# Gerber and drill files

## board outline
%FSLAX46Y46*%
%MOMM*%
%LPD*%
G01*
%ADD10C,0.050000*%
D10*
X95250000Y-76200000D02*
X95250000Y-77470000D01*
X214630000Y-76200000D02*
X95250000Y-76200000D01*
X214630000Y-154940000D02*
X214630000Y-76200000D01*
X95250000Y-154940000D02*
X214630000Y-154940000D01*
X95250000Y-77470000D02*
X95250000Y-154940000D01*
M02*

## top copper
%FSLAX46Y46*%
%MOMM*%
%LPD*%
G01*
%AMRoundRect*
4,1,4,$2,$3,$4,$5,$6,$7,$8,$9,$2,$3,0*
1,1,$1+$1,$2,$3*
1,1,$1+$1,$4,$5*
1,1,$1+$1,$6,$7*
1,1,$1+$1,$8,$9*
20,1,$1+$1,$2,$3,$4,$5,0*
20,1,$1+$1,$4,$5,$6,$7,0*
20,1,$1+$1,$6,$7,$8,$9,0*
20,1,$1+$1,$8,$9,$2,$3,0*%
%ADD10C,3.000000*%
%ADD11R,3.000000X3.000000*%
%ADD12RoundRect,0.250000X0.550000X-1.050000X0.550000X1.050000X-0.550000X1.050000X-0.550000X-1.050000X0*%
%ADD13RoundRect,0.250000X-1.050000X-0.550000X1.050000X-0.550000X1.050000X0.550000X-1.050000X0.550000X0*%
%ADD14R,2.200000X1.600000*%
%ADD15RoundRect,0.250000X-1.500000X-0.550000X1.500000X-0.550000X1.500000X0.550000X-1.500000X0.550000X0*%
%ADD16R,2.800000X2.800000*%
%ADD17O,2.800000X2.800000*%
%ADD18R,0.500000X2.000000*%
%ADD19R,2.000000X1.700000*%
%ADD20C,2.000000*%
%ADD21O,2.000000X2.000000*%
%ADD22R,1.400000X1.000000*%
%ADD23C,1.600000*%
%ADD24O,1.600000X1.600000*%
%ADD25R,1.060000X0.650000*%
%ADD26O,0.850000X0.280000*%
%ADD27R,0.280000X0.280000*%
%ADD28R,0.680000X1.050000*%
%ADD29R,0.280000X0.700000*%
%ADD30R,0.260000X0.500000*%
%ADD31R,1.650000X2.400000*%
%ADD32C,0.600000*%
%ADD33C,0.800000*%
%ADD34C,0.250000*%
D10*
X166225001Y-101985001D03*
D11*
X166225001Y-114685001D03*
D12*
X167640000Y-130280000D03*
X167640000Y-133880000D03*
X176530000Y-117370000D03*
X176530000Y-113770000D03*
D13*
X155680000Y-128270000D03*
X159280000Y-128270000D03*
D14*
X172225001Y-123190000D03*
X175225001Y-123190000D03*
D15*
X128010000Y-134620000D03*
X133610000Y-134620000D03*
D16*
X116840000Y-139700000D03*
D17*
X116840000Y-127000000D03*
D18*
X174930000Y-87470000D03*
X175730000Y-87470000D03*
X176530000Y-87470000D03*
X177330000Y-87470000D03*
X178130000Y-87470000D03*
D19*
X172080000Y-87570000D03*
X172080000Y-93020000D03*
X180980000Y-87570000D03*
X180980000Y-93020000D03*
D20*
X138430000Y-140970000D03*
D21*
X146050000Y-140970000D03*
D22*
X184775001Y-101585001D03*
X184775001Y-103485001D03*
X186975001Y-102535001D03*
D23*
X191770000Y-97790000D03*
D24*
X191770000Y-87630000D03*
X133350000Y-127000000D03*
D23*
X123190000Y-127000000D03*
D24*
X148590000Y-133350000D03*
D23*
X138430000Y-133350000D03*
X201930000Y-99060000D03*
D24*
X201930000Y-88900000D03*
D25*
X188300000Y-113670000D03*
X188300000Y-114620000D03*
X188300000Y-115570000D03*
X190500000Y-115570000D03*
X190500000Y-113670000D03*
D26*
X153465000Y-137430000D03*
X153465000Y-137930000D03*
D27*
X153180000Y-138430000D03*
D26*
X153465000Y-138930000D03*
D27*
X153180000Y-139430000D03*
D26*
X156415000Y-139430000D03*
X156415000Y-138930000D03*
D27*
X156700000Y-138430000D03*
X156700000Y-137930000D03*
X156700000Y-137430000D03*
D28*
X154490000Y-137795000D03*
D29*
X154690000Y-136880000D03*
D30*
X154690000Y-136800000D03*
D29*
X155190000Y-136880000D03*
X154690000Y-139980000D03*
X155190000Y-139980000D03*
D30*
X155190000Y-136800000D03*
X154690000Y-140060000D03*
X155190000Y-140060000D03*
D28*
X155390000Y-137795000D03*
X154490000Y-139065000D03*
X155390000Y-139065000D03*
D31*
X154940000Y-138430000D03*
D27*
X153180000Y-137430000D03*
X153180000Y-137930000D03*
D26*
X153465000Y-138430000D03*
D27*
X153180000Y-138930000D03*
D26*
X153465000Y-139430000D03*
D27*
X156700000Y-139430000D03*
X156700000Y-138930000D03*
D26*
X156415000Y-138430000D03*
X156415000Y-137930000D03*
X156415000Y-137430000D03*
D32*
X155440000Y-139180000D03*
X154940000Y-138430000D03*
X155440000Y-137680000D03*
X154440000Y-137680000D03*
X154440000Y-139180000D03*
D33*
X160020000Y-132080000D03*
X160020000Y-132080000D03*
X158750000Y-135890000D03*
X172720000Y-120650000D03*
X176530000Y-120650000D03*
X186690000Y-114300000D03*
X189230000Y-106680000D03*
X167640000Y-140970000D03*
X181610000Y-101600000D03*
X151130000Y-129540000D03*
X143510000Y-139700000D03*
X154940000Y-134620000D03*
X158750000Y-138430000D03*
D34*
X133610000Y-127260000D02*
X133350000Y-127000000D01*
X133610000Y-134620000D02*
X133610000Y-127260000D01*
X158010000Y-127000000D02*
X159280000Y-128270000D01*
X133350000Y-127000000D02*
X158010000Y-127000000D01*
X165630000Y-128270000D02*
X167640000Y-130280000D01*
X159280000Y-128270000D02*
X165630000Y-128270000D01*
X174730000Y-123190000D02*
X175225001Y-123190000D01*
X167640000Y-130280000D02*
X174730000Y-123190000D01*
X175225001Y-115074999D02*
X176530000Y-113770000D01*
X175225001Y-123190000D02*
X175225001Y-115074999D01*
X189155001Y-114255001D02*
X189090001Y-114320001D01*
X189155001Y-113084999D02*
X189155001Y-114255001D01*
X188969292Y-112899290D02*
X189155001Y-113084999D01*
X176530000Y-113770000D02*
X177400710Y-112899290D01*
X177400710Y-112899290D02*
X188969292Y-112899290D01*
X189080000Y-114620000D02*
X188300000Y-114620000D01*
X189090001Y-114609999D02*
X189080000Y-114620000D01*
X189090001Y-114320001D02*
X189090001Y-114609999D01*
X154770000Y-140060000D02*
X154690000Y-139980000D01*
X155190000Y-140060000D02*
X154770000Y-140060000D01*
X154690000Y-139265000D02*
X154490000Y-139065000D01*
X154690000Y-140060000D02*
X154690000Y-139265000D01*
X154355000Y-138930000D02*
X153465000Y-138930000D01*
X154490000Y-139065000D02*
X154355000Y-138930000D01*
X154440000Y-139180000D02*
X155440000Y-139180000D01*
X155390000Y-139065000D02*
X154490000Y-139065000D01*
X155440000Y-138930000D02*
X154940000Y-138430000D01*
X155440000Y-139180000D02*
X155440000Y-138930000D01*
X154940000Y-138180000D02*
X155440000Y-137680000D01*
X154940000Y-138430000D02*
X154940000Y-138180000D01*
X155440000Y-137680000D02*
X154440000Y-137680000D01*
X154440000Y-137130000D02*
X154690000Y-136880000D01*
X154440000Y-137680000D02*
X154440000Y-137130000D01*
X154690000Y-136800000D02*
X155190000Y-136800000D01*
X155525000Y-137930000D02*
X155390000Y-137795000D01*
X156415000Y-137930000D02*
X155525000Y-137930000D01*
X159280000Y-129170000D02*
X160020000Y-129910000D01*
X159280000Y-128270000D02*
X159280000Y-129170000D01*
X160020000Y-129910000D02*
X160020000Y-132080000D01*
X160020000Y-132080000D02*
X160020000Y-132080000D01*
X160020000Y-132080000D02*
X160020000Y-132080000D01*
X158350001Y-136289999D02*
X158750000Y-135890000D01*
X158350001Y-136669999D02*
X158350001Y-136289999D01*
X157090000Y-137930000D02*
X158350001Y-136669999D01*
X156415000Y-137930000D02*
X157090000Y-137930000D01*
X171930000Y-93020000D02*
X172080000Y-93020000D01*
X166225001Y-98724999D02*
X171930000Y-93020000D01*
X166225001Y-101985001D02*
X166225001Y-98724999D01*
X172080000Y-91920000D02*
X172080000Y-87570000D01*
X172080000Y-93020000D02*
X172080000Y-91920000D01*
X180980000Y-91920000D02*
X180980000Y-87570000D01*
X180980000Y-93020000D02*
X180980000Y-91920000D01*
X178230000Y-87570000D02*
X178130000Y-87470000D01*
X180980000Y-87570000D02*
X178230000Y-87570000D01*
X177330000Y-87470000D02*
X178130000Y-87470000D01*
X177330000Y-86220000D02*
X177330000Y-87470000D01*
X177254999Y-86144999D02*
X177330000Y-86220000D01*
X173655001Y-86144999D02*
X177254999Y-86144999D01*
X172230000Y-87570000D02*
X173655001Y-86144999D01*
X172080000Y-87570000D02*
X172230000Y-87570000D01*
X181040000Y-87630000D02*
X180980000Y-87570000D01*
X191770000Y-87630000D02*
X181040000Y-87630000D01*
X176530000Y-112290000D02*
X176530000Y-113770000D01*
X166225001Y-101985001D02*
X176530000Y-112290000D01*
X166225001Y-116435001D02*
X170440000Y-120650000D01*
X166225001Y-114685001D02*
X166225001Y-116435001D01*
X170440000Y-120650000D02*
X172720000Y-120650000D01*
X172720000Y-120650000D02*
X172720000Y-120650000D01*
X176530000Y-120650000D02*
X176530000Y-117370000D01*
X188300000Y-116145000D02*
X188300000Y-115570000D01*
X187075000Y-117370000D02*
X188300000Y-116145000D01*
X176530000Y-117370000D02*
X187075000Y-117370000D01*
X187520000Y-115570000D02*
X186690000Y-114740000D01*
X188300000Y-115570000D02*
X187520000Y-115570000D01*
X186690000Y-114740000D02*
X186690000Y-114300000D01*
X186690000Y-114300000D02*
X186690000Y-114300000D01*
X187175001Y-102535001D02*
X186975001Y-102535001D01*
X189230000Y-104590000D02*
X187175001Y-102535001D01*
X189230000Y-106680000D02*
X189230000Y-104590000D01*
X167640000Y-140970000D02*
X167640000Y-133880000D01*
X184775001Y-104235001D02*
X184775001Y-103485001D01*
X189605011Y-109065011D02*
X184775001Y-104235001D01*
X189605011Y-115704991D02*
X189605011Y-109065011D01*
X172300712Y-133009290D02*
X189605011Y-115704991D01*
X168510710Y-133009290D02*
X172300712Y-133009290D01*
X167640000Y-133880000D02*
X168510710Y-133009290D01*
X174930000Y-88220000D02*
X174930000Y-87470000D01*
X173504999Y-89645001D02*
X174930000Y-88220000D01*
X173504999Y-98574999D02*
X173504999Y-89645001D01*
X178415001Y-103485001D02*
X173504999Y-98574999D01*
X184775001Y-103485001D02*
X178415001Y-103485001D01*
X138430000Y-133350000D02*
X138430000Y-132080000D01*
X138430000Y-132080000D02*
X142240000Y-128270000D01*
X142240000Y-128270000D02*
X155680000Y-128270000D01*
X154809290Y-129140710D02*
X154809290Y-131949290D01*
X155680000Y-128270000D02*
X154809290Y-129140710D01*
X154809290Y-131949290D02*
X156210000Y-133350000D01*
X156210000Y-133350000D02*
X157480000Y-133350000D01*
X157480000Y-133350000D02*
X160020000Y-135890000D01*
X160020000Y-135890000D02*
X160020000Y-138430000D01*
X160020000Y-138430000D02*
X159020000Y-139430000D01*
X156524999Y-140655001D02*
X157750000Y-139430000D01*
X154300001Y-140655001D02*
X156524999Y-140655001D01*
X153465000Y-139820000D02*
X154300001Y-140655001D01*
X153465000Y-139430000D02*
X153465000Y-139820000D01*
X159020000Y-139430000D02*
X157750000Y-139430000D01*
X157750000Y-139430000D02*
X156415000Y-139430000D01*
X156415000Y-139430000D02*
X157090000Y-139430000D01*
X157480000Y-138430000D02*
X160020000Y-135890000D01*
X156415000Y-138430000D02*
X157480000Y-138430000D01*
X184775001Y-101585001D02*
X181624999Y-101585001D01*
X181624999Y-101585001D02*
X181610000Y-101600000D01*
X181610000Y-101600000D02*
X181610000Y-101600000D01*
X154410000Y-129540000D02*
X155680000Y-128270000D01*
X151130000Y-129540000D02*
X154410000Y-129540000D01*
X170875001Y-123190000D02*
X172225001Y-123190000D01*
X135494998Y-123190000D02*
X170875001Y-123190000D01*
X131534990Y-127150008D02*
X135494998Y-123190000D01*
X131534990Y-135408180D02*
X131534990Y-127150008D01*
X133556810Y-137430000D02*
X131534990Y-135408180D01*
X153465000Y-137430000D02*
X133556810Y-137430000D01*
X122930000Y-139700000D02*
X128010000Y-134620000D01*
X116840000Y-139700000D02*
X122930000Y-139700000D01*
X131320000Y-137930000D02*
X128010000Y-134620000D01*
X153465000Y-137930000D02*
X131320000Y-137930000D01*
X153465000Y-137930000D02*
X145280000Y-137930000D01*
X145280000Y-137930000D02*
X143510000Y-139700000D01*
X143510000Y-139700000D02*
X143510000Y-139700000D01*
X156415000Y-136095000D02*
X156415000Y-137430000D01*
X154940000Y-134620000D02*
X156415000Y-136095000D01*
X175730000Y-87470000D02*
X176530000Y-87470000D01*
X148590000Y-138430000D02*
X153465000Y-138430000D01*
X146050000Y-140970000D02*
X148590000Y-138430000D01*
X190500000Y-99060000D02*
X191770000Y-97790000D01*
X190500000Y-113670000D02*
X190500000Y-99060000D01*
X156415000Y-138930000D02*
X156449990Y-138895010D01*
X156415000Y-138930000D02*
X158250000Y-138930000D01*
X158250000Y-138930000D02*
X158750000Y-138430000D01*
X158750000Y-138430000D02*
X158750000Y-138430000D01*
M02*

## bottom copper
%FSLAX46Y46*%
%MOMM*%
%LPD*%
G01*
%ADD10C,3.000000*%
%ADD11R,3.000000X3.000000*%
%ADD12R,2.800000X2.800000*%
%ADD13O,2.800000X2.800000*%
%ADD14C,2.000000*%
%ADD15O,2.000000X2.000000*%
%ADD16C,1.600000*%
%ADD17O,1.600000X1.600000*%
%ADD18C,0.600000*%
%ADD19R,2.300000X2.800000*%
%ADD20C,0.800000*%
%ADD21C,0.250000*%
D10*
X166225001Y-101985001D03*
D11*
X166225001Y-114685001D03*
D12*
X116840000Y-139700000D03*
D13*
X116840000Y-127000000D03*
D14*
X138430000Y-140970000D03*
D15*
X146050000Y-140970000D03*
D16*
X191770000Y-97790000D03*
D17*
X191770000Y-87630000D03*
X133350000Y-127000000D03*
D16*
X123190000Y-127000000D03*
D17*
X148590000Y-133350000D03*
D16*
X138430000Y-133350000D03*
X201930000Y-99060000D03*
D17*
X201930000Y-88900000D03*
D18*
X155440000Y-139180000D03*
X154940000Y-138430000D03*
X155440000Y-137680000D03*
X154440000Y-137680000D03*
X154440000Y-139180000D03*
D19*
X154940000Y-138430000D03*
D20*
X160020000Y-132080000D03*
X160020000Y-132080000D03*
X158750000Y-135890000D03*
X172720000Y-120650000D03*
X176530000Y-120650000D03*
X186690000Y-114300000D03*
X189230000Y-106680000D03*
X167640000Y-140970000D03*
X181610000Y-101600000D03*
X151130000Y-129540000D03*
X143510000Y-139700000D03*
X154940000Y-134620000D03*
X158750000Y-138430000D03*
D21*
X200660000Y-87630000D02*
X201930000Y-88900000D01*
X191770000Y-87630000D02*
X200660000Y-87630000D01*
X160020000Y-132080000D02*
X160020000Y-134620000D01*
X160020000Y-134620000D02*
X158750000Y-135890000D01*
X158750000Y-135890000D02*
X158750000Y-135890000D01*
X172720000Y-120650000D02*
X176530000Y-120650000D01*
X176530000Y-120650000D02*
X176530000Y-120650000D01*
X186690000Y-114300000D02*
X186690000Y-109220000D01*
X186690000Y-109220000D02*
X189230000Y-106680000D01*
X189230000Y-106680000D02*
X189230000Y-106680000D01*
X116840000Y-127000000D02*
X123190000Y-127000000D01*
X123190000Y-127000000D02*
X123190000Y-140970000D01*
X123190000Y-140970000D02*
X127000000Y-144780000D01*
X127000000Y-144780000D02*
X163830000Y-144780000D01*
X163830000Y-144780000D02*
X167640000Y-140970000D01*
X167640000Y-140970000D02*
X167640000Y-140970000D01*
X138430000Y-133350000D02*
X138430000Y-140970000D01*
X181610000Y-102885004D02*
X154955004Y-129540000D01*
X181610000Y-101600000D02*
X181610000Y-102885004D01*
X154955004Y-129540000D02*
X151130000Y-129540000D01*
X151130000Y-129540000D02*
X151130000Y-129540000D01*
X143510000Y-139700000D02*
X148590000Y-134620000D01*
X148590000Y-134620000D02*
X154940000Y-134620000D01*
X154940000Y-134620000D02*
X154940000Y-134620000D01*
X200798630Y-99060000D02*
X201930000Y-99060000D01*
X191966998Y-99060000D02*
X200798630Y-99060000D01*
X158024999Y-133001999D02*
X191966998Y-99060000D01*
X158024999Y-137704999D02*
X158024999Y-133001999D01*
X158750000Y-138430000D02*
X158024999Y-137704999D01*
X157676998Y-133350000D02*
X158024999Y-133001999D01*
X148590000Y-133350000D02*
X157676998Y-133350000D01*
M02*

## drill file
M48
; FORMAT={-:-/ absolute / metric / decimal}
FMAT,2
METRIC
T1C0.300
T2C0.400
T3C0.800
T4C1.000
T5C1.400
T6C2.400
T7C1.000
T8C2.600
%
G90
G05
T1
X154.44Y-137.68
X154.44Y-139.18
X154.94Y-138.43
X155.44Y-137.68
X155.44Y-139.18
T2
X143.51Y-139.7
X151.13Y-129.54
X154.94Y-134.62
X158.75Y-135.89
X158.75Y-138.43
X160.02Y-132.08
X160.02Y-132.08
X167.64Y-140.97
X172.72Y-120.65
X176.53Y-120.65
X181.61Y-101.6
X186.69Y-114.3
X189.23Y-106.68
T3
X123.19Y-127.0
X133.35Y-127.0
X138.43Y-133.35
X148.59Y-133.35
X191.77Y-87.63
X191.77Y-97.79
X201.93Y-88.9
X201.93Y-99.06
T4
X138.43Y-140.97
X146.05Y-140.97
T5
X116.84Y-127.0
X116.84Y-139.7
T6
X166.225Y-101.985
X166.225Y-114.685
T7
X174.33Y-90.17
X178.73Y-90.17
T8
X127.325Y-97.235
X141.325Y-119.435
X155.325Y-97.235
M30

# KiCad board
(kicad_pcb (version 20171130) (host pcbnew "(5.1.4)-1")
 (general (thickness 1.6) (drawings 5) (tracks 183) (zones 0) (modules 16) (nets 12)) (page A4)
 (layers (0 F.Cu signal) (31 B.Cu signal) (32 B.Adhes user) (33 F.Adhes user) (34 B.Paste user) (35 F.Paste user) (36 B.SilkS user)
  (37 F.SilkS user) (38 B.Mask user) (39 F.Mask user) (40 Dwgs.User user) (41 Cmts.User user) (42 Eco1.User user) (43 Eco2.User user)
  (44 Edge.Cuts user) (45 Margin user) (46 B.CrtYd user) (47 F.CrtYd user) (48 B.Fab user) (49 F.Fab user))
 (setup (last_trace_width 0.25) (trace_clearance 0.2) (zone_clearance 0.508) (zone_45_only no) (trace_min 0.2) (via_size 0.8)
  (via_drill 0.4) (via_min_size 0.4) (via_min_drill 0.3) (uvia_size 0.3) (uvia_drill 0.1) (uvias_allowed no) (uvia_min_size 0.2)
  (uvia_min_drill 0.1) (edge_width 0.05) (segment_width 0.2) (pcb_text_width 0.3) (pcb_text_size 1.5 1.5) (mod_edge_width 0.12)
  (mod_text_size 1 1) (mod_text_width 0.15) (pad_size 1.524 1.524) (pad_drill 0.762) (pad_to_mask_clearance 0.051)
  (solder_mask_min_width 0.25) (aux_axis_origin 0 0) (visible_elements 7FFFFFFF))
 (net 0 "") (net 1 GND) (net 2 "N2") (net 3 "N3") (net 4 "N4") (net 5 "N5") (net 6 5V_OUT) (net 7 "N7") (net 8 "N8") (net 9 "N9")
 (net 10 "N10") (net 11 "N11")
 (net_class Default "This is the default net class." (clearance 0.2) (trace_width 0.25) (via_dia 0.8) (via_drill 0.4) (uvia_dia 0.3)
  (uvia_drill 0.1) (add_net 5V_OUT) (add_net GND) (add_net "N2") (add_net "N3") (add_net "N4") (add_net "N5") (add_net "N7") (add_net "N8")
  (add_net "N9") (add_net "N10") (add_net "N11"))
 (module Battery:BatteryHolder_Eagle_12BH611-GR (layer F.Cu) (at 166.225001 114.685001)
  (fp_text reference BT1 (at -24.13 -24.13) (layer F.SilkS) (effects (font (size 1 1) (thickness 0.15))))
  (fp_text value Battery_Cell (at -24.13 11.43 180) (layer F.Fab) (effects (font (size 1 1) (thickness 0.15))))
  (pad 2 thru_hole circle (at 0 -12.7) (size 3 3) (drill 2.4) (layers *.Cu *.Mask) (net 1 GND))
  (pad 1 thru_hole rect (at 0 0) (size 3 3) (drill 2.4) (layers *.Cu *.Mask) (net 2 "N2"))
  (pad "" np_thru_hole circle (at -10.9 -17.45) (size 2.6 2.6) (drill 2.6) (layers *.Cu *.Mask))
  (pad "" np_thru_hole circle (at -38.9 -17.45) (size 2.6 2.6) (drill 2.6) (layers *.Cu *.Mask))
  (pad "" np_thru_hole circle (at -24.9 4.75) (size 2.6 2.6) (drill 2.6) (layers *.Cu *.Mask)))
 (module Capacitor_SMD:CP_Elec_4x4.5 (layer F.Cu) (at 167.64 132.08 90)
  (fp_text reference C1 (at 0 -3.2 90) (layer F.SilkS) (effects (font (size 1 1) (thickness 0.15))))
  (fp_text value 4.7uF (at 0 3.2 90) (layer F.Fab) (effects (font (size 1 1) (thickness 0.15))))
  (pad 2 smd roundrect (at 1.8 0 90) (size 2.6 1.6) (layers F.Cu F.Paste F.Mask) (roundrect_rratio 0.15625) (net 1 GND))
  (pad 1 smd roundrect (at -1.8 0 90) (size 2.6 1.6) (layers F.Cu F.Paste F.Mask) (roundrect_rratio 0.15625) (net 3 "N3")))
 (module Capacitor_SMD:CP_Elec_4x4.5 (layer F.Cu) (at 176.53 115.57 90)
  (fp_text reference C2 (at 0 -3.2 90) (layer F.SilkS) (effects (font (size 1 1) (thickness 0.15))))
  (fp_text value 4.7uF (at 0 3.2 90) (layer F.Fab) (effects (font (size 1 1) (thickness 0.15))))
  (pad 1 smd roundrect (at -1.8 0 90) (size 2.6 1.6) (layers F.Cu F.Paste F.Mask) (roundrect_rratio 0.15625) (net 2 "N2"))
  (pad 2 smd roundrect (at 1.8 0 90) (size 2.6 1.6) (layers F.Cu F.Paste F.Mask) (roundrect_rratio 0.15625) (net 1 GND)))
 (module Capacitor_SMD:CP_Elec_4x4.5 (layer F.Cu) (at 157.48 128.27)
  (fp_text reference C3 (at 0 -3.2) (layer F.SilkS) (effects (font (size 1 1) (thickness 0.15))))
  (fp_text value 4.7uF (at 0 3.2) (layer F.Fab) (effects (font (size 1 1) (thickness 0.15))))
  (pad 1 smd roundrect (at -1.8 0) (size 2.6 1.6) (layers F.Cu F.Paste F.Mask) (roundrect_rratio 0.15625) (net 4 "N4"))
  (pad 2 smd roundrect (at 1.8 0) (size 2.6 1.6) (layers F.Cu F.Paste F.Mask) (roundrect_rratio 0.15625) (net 1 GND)))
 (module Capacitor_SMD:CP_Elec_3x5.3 (layer F.Cu) (at 173.725001 123.19)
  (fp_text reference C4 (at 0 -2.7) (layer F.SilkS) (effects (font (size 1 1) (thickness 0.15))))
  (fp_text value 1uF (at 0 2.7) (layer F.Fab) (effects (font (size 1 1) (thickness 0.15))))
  (pad 1 smd rect (at -1.5 0) (size 2.2 1.6) (layers F.Cu F.Paste F.Mask) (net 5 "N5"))
  (pad 2 smd rect (at 1.5 0) (size 2.2 1.6) (layers F.Cu F.Paste F.Mask) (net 1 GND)))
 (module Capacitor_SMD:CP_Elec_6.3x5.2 (layer F.Cu) (at 130.81 134.62)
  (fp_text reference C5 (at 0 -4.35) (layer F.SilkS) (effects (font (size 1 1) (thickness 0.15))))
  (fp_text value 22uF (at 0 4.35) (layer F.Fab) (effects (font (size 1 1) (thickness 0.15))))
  (pad 1 smd roundrect (at -2.8 0) (size 3.5 1.6) (layers F.Cu F.Paste F.Mask) (roundrect_rratio 0.15625) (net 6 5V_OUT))
  (pad 2 smd roundrect (at 2.8 0) (size 3.5 1.6) (layers F.Cu F.Paste F.Mask) (roundrect_rratio 0.15625) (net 1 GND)))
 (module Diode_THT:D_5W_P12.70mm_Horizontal (layer F.Cu) (at 116.84 139.7 90)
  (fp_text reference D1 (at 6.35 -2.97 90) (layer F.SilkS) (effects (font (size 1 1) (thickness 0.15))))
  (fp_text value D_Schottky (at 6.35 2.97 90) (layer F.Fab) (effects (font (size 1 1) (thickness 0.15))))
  (pad 1 thru_hole rect (at 0 0 90) (size 2.8 2.8) (drill 1.4) (layers *.Cu *.Mask) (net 6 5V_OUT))
  (pad 2 thru_hole oval (at 12.7 0 90) (size 2.8 2.8) (drill 1.4) (layers *.Cu *.Mask) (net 3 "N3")))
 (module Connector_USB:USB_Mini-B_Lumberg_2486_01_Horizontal (layer F.Cu) (at 176.53 90.17)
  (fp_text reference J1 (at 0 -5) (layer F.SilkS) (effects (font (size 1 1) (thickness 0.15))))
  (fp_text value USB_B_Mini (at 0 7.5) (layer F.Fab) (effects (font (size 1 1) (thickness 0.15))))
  (pad 1 smd rect (at -1.6 -2.7) (size 0.5 2) (layers F.Cu F.Paste F.Mask) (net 3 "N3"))
  (pad 2 smd rect (at -0.8 -2.7) (size 0.5 2) (layers F.Cu F.Paste F.Mask) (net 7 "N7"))
  (pad 3 smd rect (at 0 -2.7) (size 0.5 2) (layers F.Cu F.Paste F.Mask) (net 7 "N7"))
  (pad 4 smd rect (at 0.8 -2.7) (size 0.5 2) (layers F.Cu F.Paste F.Mask) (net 1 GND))
  (pad 5 smd rect (at 1.6 -2.7) (size 0.5 2) (layers F.Cu F.Paste F.Mask) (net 1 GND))
  (pad 6 smd rect (at -4.45 -2.6) (size 2 1.7) (layers F.Cu F.Paste F.Mask) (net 1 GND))
  (pad 6 smd rect (at -4.45 2.85) (size 2 1.7) (layers F.Cu F.Paste F.Mask) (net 1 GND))
  (pad 6 smd rect (at 4.45 -2.6) (size 2 1.7) (layers F.Cu F.Paste F.Mask) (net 1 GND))
  (pad 6 smd rect (at 4.45 2.85) (size 2 1.7) (layers F.Cu F.Paste F.Mask) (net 1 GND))
  (pad "" np_thru_hole circle (at -2.2 0) (size 1 1) (drill 1) (layers *.Cu *.Mask))
  (pad "" np_thru_hole circle (at 2.2 0) (size 1 1) (drill 1) (layers *.Cu *.Mask)))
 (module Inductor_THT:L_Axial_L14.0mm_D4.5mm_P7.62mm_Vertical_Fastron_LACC (layer F.Cu) (at 138.43 140.97)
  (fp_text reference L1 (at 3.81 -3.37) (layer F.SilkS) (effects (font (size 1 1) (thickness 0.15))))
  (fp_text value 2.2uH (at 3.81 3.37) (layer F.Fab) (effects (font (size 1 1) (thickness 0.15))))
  (pad 1 thru_hole circle (at 0 0) (size 2 2) (drill 1) (layers *.Cu *.Mask) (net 4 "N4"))
  (pad 2 thru_hole oval (at 7.62 0) (size 2 2) (drill 1) (layers *.Cu *.Mask) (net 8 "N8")))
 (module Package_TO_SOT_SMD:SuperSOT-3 (layer F.Cu) (at 185.875001 102.535001)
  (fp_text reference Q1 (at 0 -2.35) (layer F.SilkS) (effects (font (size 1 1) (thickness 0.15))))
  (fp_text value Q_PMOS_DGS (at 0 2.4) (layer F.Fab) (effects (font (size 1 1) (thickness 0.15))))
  (pad 1 smd rect (at -1.1 -0.95) (size 1.4 1) (layers F.Cu F.Paste F.Mask) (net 4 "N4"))
  (pad 2 smd rect (at -1.1 0.95) (size 1.4 1) (layers F.Cu F.Paste F.Mask) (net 3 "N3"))
  (pad 3 smd rect (at 1.1 0) (size 1.4 1) (layers F.Cu F.Paste F.Mask) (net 2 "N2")))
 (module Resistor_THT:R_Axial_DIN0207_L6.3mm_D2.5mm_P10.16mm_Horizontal (layer F.Cu) (at 191.77 97.79 90)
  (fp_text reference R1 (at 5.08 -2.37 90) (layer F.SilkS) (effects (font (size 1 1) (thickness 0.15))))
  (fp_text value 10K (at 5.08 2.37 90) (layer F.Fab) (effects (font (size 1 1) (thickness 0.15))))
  (pad 1 thru_hole circle (at 0 0 90) (size 1.6 1.6) (drill 0.8) (layers *.Cu *.Mask) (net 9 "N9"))
  (pad 2 thru_hole oval (at 10.16 0 90) (size 1.6 1.6) (drill 0.8) (layers *.Cu *.Mask) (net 1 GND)))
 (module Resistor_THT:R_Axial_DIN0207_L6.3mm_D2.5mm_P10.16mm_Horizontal (layer F.Cu) (at 123.19 127)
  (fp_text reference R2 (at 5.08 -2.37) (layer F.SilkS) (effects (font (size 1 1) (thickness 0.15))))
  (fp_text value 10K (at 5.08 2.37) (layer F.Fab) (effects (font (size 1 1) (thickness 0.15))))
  (pad 2 thru_hole oval (at 10.16 0) (size 1.6 1.6) (drill 0.8) (layers *.Cu *.Mask) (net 1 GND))
  (pad 1 thru_hole circle (at 0 0) (size 1.6 1.6) (drill 0.8) (layers *.Cu *.Mask) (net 3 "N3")))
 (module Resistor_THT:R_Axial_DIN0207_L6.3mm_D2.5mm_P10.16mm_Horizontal (layer F.Cu) (at 138.43 133.35)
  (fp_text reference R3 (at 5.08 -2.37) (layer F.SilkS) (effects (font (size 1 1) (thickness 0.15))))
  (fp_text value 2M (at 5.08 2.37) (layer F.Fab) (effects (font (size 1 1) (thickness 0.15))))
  (pad 2 thru_hole oval (at 10.16 0) (size 1.6 1.6) (drill 0.8) (layers *.Cu *.Mask) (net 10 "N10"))
  (pad 1 thru_hole circle (at 0 0) (size 1.6 1.6) (drill 0.8) (layers *.Cu *.Mask) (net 4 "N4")))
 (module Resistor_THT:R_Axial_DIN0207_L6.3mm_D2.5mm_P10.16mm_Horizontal (layer F.Cu) (at 201.93 99.06 90)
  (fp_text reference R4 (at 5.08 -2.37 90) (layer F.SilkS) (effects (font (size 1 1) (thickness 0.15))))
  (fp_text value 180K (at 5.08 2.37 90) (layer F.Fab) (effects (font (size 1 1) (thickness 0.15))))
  (pad 1 thru_hole circle (at 0 0 90) (size 1.6 1.6) (drill 0.8) (layers *.Cu *.Mask) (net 10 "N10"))
  (pad 2 thru_hole oval (at 10.16 0 90) (size 1.6 1.6) (drill 0.8) (layers *.Cu *.Mask) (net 1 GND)))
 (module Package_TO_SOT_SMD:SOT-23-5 (layer F.Cu) (at 189.4 114.62)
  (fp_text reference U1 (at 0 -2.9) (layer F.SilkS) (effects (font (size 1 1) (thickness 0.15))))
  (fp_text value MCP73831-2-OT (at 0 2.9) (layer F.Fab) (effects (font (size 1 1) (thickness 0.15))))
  (pad 1 smd rect (at -1.1 -0.95) (size 1.06 0.65) (layers F.Cu F.Paste F.Mask) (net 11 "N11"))
  (pad 2 smd rect (at -1.1 0) (size 1.06 0.65) (layers F.Cu F.Paste F.Mask) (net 1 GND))
  (pad 3 smd rect (at -1.1 0.95) (size 1.06 0.65) (layers F.Cu F.Paste F.Mask) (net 2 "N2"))
  (pad 4 smd rect (at 1.1 0.95) (size 1.06 0.65) (layers F.Cu F.Paste F.Mask) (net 3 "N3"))
  (pad 5 smd rect (at 1.1 -0.95) (size 1.06 0.65) (layers F.Cu F.Paste F.Mask) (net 9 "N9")))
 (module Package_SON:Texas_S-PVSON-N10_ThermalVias (layer F.Cu) (at 154.94 138.43)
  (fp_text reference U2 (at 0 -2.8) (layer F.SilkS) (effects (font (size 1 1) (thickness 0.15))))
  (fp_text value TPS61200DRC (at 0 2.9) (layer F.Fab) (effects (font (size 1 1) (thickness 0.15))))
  (pad 1 smd oval (at -1.475 -1) (size 0.85 0.28) (layers F.Cu F.Paste F.Mask) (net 5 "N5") (solder_mask_margin 0.07)
   (solder_paste_margin -0.025))
  (pad 2 smd oval (at -1.475 -0.5) (size 0.85 0.28) (layers F.Cu F.Paste F.Mask) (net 6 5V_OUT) (solder_mask_margin 0.07)
   (solder_paste_margin -0.025))
  (pad 3 smd rect (at -1.76 0) (size 0.28 0.28) (layers F.Cu F.Paste F.Mask) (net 8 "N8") (solder_mask_margin 0.07)
   (solder_paste_margin -0.025))
  (pad 4 smd oval (at -1.475 0.5) (size 0.85 0.28) (layers F.Cu F.Paste F.Mask) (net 1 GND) (solder_mask_margin 0.07)
   (solder_paste_margin -0.025))
  (pad 5 smd rect (at -1.76 1) (size 0.28 0.28) (layers F.Cu F.Paste F.Mask) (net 4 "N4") (solder_mask_margin 0.07)
   (solder_paste_margin -0.025))
  (pad 6 smd oval (at 1.475 1) (size 0.85 0.28) (layers F.Cu F.Paste F.Mask) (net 4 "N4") (solder_mask_margin 0.07)
   (solder_paste_margin -0.025))
  (pad 7 smd oval (at 1.475 0.5) (size 0.85 0.28) (layers F.Cu F.Paste F.Mask) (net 10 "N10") (solder_mask_margin 0.07)
   (solder_paste_margin -0.025))
  (pad 8 smd rect (at 1.76 0) (size 0.28 0.28) (layers F.Cu F.Paste F.Mask) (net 4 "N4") (solder_mask_margin 0.07)
   (solder_paste_margin -0.025))
  (pad 9 smd rect (at 1.76 -0.5) (size 0.28 0.28) (layers F.Cu F.Paste F.Mask) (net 1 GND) (solder_mask_margin 0.07)
   (solder_paste_margin -0.025))
  (pad 10 smd rect (at 1.76 -1) (size 0.28 0.28) (layers F.Cu F.Paste F.Mask) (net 6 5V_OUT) (solder_mask_margin 0.07)
   (solder_paste_margin -0.025))
  (pad 11 smd rect (at -0.45 -0.635) (size 0.68 1.05) (layers F.Cu F.Paste F.Mask) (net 1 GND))
  (pad 11 smd rect (at -0.25 -1.55) (size 0.28 0.7) (layers F.Cu F.Mask) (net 1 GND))
  (pad 11 smd rect (at -0.25 -1.63) (size 0.26 0.5) (layers F.Cu F.Paste F.Mask) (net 1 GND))
  (pad 11 smd rect (at 0.25 -1.55) (size 0.28 0.7) (layers F.Cu F.Mask) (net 1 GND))
  (pad 11 smd rect (at -0.25 1.55) (size 0.28 0.7) (layers F.Cu F.Mask) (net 1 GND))
  (pad 11 smd rect (at 0.25 1.55) (size 0.28 0.7) (layers F.Cu F.Mask) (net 1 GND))
  (pad 11 smd rect (at 0.25 -1.63) (size 0.26 0.5) (layers F.Cu F.Paste F.Mask) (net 1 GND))
  (pad 11 smd rect (at -0.25 1.63) (size 0.26 0.5) (layers F.Cu F.Paste F.Mask) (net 1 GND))
  (pad 11 smd rect (at 0.25 1.63) (size 0.26 0.5) (layers F.Cu F.Paste F.Mask) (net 1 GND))
  (pad 11 smd rect (at 0.45 -0.635) (size 0.68 1.05) (layers F.Cu F.Paste F.Mask) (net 1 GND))
  (pad 11 smd rect (at -0.45 0.635) (size 0.68 1.05) (layers F.Cu F.Paste F.Mask) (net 1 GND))
  (pad 11 smd rect (at 0.45 0.635) (size 0.68 1.05) (layers F.Cu F.Paste F.Mask) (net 1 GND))
  (pad 11 smd rect (at 0 0) (size 1.65 2.4) (layers F.Cu F.Mask) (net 1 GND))
  (pad 1 smd rect (at -1.76 -1) (size 0.28 0.28) (layers F.Cu F.Paste F.Mask) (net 5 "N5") (solder_mask_margin 0.07)
   (solder_paste_margin -0.025))
  (pad 2 smd rect (at -1.76 -0.5) (size 0.28 0.28) (layers F.Cu F.Paste F.Mask) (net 6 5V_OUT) (solder_mask_margin 0.07)
   (solder_paste_margin -0.025))
  (pad 3 smd oval (at -1.475 0) (size 0.85 0.28) (layers F.Cu F.Paste F.Mask) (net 8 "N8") (solder_mask_margin 0.07)
   (solder_paste_margin -0.025))
  (pad 4 smd rect (at -1.76 0.5) (size 0.28 0.28) (layers F.Cu F.Paste F.Mask) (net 1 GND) (solder_mask_margin 0.07)
   (solder_paste_margin -0.025))
  (pad 5 smd oval (at -1.475 1) (size 0.85 0.28) (layers F.Cu F.Paste F.Mask) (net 4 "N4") (solder_mask_margin 0.07)
   (solder_paste_margin -0.025))
  (pad 6 smd rect (at 1.76 1) (size 0.28 0.28) (layers F.Cu F.Paste F.Mask) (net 4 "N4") (solder_mask_margin 0.07)
   (solder_paste_margin -0.025))
  (pad 7 smd rect (at 1.76 0.5) (size 0.28 0.28) (layers F.Cu F.Paste F.Mask) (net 10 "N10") (solder_mask_margin 0.07)
   (solder_paste_margin -0.025))
  (pad 8 smd oval (at 1.475 0) (size 0.85 0.28) (layers F.Cu F.Paste F.Mask) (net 4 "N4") (solder_mask_margin 0.07)
   (solder_paste_margin -0.025))
  (pad 9 smd oval (at 1.475 -0.5) (size 0.85 0.28) (layers F.Cu F.Paste F.Mask) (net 1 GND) (solder_mask_margin 0.07)
   (solder_paste_margin -0.025))
  (pad 10 smd oval (at 1.475 -1) (size 0.85 0.28) (layers F.Cu F.Paste F.Mask) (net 6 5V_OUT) (solder_mask_margin 0.07)
   (solder_paste_margin -0.025))
  (pad 11 thru_hole circle (at 0.5 0.75) (size 0.6 0.6) (drill 0.3) (layers *.Cu *.Mask) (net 1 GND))
  (pad 11 thru_hole circle (at 0 0) (size 0.6 0.6) (drill 0.3) (layers *.Cu *.Mask) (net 1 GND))
  (pad 11 thru_hole circle (at 0.5 -0.75) (size 0.6 0.6) (drill 0.3) (layers *.Cu *.Mask) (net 1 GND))
  (pad 11 thru_hole circle (at -0.5 -0.75) (size 0.6 0.6) (drill 0.3) (layers *.Cu *.Mask) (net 1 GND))
  (pad 11 thru_hole circle (at -0.5 0.75) (size 0.6 0.6) (drill 0.3) (layers *.Cu *.Mask) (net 1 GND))
  (pad 11 smd rect (at 0 0) (size 2.3 2.8) (layers B.Cu) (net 1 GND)))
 (gr_line (start 95.25 76.2) (end 95.25 77.47) (layer Edge.Cuts) (width 0.05))
 (gr_line (start 214.63 76.2) (end 95.25 76.2) (layer Edge.Cuts) (width 0.05))
 (gr_line (start 214.63 154.94) (end 214.63 76.2) (layer Edge.Cuts) (width 0.05))
 (gr_line (start 95.25 154.94) (end 214.63 154.94) (layer Edge.Cuts) (width 0.05))
 (gr_line (start 95.25 77.47) (end 95.25 154.94) (layer Edge.Cuts) (width 0.05))
 (segment (start 200.66 87.63) (end 201.93 88.9) (width 0.25) (layer B.Cu) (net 1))
 (segment (start 191.77 87.63) (end 200.66 87.63) (width 0.25) (layer B.Cu) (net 1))
 (segment (start 133.61 127.26) (end 133.35 127) (width 0.25) (layer F.Cu) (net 1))
 (segment (start 133.61 134.62) (end 133.61 127.26) (width 0.25) (layer F.Cu) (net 1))
 (segment (start 158.01 127) (end 159.28 128.27) (width 0.25) (layer F.Cu) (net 1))
 (segment (start 133.35 127) (end 158.01 127) (width 0.25) (layer F.Cu) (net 1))
 (segment (start 165.63 128.27) (end 167.64 130.28) (width 0.25) (layer F.Cu) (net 1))
 (segment (start 159.28 128.27) (end 165.63 128.27) (width 0.25) (layer F.Cu) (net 1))
 (segment (start 174.73 123.19) (end 175.225001 123.19) (width 0.25) (layer F.Cu) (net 1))
 (segment (start 167.64 130.28) (end 174.73 123.19) (width 0.25) (layer F.Cu) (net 1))
 (segment (start 175.225001 115.074999) (end 176.53 113.77) (width 0.25) (layer F.Cu) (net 1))
 (segment (start 175.225001 123.19) (end 175.225001 115.074999) (width 0.25) (layer F.Cu) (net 1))
 (segment (start 189.155001 114.255001) (end 189.090001 114.320001) (width 0.25) (layer F.Cu) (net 1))
 (segment (start 189.155001 113.084999) (end 189.155001 114.255001) (width 0.25) (layer F.Cu) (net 1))
 (segment (start 188.969292 112.89929) (end 189.155001 113.084999) (width 0.25) (layer F.Cu) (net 1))
 (segment (start 176.53 113.77) (end 177.40071 112.89929) (width 0.25) (layer F.Cu) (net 1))
 (segment (start 177.40071 112.89929) (end 188.969292 112.89929) (width 0.25) (layer F.Cu) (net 1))
 (segment (start 189.08 114.62) (end 188.3 114.62) (width 0.25) (layer F.Cu) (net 1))
 (segment (start 189.090001 114.609999) (end 189.08 114.62) (width 0.25) (layer F.Cu) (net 1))
 (segment (start 189.090001 114.320001) (end 189.090001 114.609999) (width 0.25) (layer F.Cu) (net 1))
 (segment (start 154.77 140.06) (end 154.69 139.98) (width 0.25) (layer F.Cu) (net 1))
 (segment (start 155.19 140.06) (end 154.77 140.06) (width 0.25) (layer F.Cu) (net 1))
 (segment (start 154.69 139.265) (end 154.49 139.065) (width 0.25) (layer F.Cu) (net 1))
 (segment (start 154.69 140.06) (end 154.69 139.265) (width 0.25) (layer F.Cu) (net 1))
 (segment (start 154.355 138.93) (end 153.465 138.93) (width 0.25) (layer F.Cu) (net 1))
 (segment (start 154.49 139.065) (end 154.355 138.93) (width 0.25) (layer F.Cu) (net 1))
 (segment (start 154.44 139.18) (end 155.44 139.18) (width 0.25) (layer F.Cu) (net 1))
 (segment (start 155.39 139.065) (end 154.49 139.065) (width 0.25) (layer F.Cu) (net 1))
 (segment (start 155.44 138.93) (end 154.94 138.43) (width 0.25) (layer F.Cu) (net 1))
 (segment (start 155.44 139.18) (end 155.44 138.93) (width 0.25) (layer F.Cu) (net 1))
 (segment (start 154.94 138.18) (end 155.44 137.68) (width 0.25) (layer F.Cu) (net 1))
 (segment (start 154.94 138.43) (end 154.94 138.18) (width 0.25) (layer F.Cu) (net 1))
 (segment (start 155.44 137.68) (end 154.44 137.68) (width 0.25) (layer F.Cu) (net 1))
 (segment (start 154.44 137.13) (end 154.69 136.88) (width 0.25) (layer F.Cu) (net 1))
 (segment (start 154.44 137.68) (end 154.44 137.13) (width 0.25) (layer F.Cu) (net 1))
 (segment (start 154.69 136.8) (end 155.19 136.8) (width 0.25) (layer F.Cu) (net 1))
 (segment (start 155.525 137.93) (end 155.39 137.795) (width 0.25) (layer F.Cu) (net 1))
 (segment (start 156.415 137.93) (end 155.525 137.93) (width 0.25) (layer F.Cu) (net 1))
 (segment (start 159.28 129.17) (end 160.02 129.91) (width 0.25) (layer F.Cu) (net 1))
 (segment (start 159.28 128.27) (end 159.28 129.17) (width 0.25) (layer F.Cu) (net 1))
 (segment (start 160.02 129.91) (end 160.02 132.08) (width 0.25) (layer F.Cu) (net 1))
 (segment (start 160.02 132.08) (end 160.02 132.08) (width 0.25) (layer F.Cu) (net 1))
 (via (at 160.02 132.08) (size 0.8) (drill 0.4) (layers F.Cu B.Cu) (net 1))
 (segment (start 160.02 132.08) (end 160.02 132.08) (width 0.25) (layer F.Cu) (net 1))
 (via (at 160.02 132.08) (size 0.8) (drill 0.4) (layers F.Cu B.Cu) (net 1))
 (segment (start 160.02 132.08) (end 160.02 134.62) (width 0.25) (layer B.Cu) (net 1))
 (segment (start 160.02 134.62) (end 158.75 135.89) (width 0.25) (layer B.Cu) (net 1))
 (segment (start 158.75 135.89) (end 158.75 135.89) (width 0.25) (layer B.Cu) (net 1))
 (via (at 158.75 135.89) (size 0.8) (drill 0.4) (layers F.Cu B.Cu) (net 1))
 (segment (start 158.350001 136.289999) (end 158.75 135.89) (width 0.25) (layer F.Cu) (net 1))
 (segment (start 158.350001 136.669999) (end 158.350001 136.289999) (width 0.25) (layer F.Cu) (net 1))
 (segment (start 157.09 137.93) (end 158.350001 136.669999) (width 0.25) (layer F.Cu) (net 1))
 (segment (start 156.415 137.93) (end 157.09 137.93) (width 0.25) (layer F.Cu) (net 1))
 (segment (start 171.93 93.02) (end 172.08 93.02) (width 0.25) (layer F.Cu) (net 1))
 (segment (start 166.225001 98.724999) (end 171.93 93.02) (width 0.25) (layer F.Cu) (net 1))
 (segment (start 166.225001 101.985001) (end 166.225001 98.724999) (width 0.25) (layer F.Cu) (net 1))
 (segment (start 172.08 91.92) (end 172.08 87.57) (width 0.25) (layer F.Cu) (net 1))
 (segment (start 172.08 93.02) (end 172.08 91.92) (width 0.25) (layer F.Cu) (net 1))
 (segment (start 180.98 91.92) (end 180.98 87.57) (width 0.25) (layer F.Cu) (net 1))
 (segment (start 180.98 93.02) (end 180.98 91.92) (width 0.25) (layer F.Cu) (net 1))
 (segment (start 178.23 87.57) (end 178.13 87.47) (width 0.25) (layer F.Cu) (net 1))
 (segment (start 180.98 87.57) (end 178.23 87.57) (width 0.25) (layer F.Cu) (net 1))
 (segment (start 177.33 87.47) (end 178.13 87.47) (width 0.25) (layer F.Cu) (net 1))
 (segment (start 177.33 86.22) (end 177.33 87.47) (width 0.25) (layer F.Cu) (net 1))
 (segment (start 177.254999 86.144999) (end 177.33 86.22) (width 0.25) (layer F.Cu) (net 1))
 (segment (start 173.655001 86.144999) (end 177.254999 86.144999) (width 0.25) (layer F.Cu) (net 1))
 (segment (start 172.23 87.57) (end 173.655001 86.144999) (width 0.25) (layer F.Cu) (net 1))
 (segment (start 172.08 87.57) (end 172.23 87.57) (width 0.25) (layer F.Cu) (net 1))
 (segment (start 181.04 87.63) (end 180.98 87.57) (width 0.25) (layer F.Cu) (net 1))
 (segment (start 191.77 87.63) (end 181.04 87.63) (width 0.25) (layer F.Cu) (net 1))
 (segment (start 176.53 112.29) (end 176.53 113.77) (width 0.25) (layer F.Cu) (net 1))
 (segment (start 166.225001 101.985001) (end 176.53 112.29) (width 0.25) (layer F.Cu) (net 1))
 (segment (start 166.225001 116.435001) (end 170.44 120.65) (width 0.25) (layer F.Cu) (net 2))
 (segment (start 166.225001 114.685001) (end 166.225001 116.435001) (width 0.25) (layer F.Cu) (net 2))
 (segment (start 170.44 120.65) (end 172.72 120.65) (width 0.25) (layer F.Cu) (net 2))
 (segment (start 172.72 120.65) (end 172.72 120.65) (width 0.25) (layer F.Cu) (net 2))
 (via (at 172.72 120.65) (size 0.8) (drill 0.4) (layers F.Cu B.Cu) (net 2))
 (segment (start 172.72 120.65) (end 176.53 120.65) (width 0.25) (layer B.Cu) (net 2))
 (segment (start 176.53 120.65) (end 176.53 120.65) (width 0.25) (layer B.Cu) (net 2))
 (via (at 176.53 120.65) (size 0.8) (drill 0.4) (layers F.Cu B.Cu) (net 2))
 (segment (start 176.53 120.65) (end 176.53 117.37) (width 0.25) (layer F.Cu) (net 2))
 (segment (start 188.3 116.145) (end 188.3 115.57) (width 0.25) (layer F.Cu) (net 2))
 (segment (start 187.075 117.37) (end 188.3 116.145) (width 0.25) (layer F.Cu) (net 2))
 (segment (start 176.53 117.37) (end 187.075 117.37) (width 0.25) (layer F.Cu) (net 2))
 (segment (start 187.52 115.57) (end 186.69 114.74) (width 0.25) (layer F.Cu) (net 2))
 (segment (start 188.3 115.57) (end 187.52 115.57) (width 0.25) (layer F.Cu) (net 2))
 (segment (start 186.69 114.74) (end 186.69 114.3) (width 0.25) (layer F.Cu) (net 2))
 (segment (start 186.69 114.3) (end 186.69 114.3) (width 0.25) (layer F.Cu) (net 2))
 (via (at 186.69 114.3) (size 0.8) (drill 0.4) (layers F.Cu B.Cu) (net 2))
 (segment (start 186.69 114.3) (end 186.69 109.22) (width 0.25) (layer B.Cu) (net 2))
 (segment (start 186.69 109.22) (end 189.23 106.68) (width 0.25) (layer B.Cu) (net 2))
 (segment (start 189.23 106.68) (end 189.23 106.68) (width 0.25) (layer B.Cu) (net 2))
 (via (at 189.23 106.68) (size 0.8) (drill 0.4) (layers F.Cu B.Cu) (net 2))
 (segment (start 187.175001 102.535001) (end 186.975001 102.535001) (width 0.25) (layer F.Cu) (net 2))
 (segment (start 189.23 104.59) (end 187.175001 102.535001) (width 0.25) (layer F.Cu) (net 2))
 (segment (start 189.23 106.68) (end 189.23 104.59) (width 0.25) (layer F.Cu) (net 2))
 (segment (start 116.84 127) (end 123.19 127) (width 0.25) (layer B.Cu) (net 3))
 (segment (start 123.19 127) (end 123.19 140.97) (width 0.25) (layer B.Cu) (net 3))
 (segment (start 123.19 140.97) (end 127 144.78) (width 0.25) (layer B.Cu) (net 3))
 (segment (start 127 144.78) (end 163.83 144.78) (width 0.25) (layer B.Cu) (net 3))
 (segment (start 163.83 144.78) (end 167.64 140.97) (width 0.25) (layer B.Cu) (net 3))
 (segment (start 167.64 140.97) (end 167.64 140.97) (width 0.25) (layer B.Cu) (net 3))
 (via (at 167.64 140.97) (size 0.8) (drill 0.4) (layers F.Cu B.Cu) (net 3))
 (segment (start 167.64 140.97) (end 167.64 133.88) (width 0.25) (layer F.Cu) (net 3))
 (segment (start 184.775001 104.235001) (end 184.775001 103.485001) (width 0.25) (layer F.Cu) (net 3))
 (segment (start 189.605011 109.065011) (end 184.775001 104.235001) (width 0.25) (layer F.Cu) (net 3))
 (segment (start 189.605011 115.704991) (end 189.605011 109.065011) (width 0.25) (layer F.Cu) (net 3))
 (segment (start 172.300712 133.00929) (end 189.605011 115.704991) (width 0.25) (layer F.Cu) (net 3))
 (segment (start 168.51071 133.00929) (end 172.300712 133.00929) (width 0.25) (layer F.Cu) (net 3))
 (segment (start 167.64 133.88) (end 168.51071 133.00929) (width 0.25) (layer F.Cu) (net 3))
 (segment (start 174.93 88.22) (end 174.93 87.47) (width 0.25) (layer F.Cu) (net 3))
 (segment (start 173.504999 89.645001) (end 174.93 88.22) (width 0.25) (layer F.Cu) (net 3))
 (segment (start 173.504999 98.574999) (end 173.504999 89.645001) (width 0.25) (layer F.Cu) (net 3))
 (segment (start 178.415001 103.485001) (end 173.504999 98.574999) (width 0.25) (layer F.Cu) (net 3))
 (segment (start 184.775001 103.485001) (end 178.415001 103.485001) (width 0.25) (layer F.Cu) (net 3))
 (segment (start 138.43 133.35) (end 138.43 140.97) (width 0.25) (layer B.Cu) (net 4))
 (segment (start 138.43 133.35) (end 138.43 132.08) (width 0.25) (layer F.Cu) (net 4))
 (segment (start 138.43 132.08) (end 142.24 128.27) (width 0.25) (layer F.Cu) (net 4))
 (segment (start 142.24 128.27) (end 155.68 128.27) (width 0.25) (layer F.Cu) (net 4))
 (segment (start 154.80929 129.14071) (end 154.80929 131.94929) (width 0.25) (layer F.Cu) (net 4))
 (segment (start 155.68 128.27) (end 154.80929 129.14071) (width 0.25) (layer F.Cu) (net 4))
 (segment (start 154.80929 131.94929) (end 156.21 133.35) (width 0.25) (layer F.Cu) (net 4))
 (segment (start 156.21 133.35) (end 157.48 133.35) (width 0.25) (layer F.Cu) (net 4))
 (segment (start 157.48 133.35) (end 160.02 135.89) (width 0.25) (layer F.Cu) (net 4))
 (segment (start 160.02 135.89) (end 160.02 138.43) (width 0.25) (layer F.Cu) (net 4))
 (segment (start 160.02 138.43) (end 159.02 139.43) (width 0.25) (layer F.Cu) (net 4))
 (segment (start 156.524999 140.655001) (end 157.75 139.43) (width 0.25) (layer F.Cu) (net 4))
 (segment (start 154.300001 140.655001) (end 156.524999 140.655001) (width 0.25) (layer F.Cu) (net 4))
 (segment (start 153.465 139.82) (end 154.300001 140.655001) (width 0.25) (layer F.Cu) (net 4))
 (segment (start 153.465 139.43) (end 153.465 139.82) (width 0.25) (layer F.Cu) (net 4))
 (segment (start 159.02 139.43) (end 157.75 139.43) (width 0.25) (layer F.Cu) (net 4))
 (segment (start 157.75 139.43) (end 156.415 139.43) (width 0.25) (layer F.Cu) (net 4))
 (segment (start 156.415 139.43) (end 157.09 139.43) (width 0.25) (layer F.Cu) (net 4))
 (segment (start 157.48 138.43) (end 160.02 135.89) (width 0.25) (layer F.Cu) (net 4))
 (segment (start 156.415 138.43) (end 157.48 138.43) (width 0.25) (layer F.Cu) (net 4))
 (segment (start 184.775001 101.585001) (end 181.624999 101.585001) (width 0.25) (layer F.Cu) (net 4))
 (segment (start 181.624999 101.585001) (end 181.61 101.6) (width 0.25) (layer F.Cu) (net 4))
 (segment (start 181.61 101.6) (end 181.61 101.6) (width 0.25) (layer F.Cu) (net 4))
 (via (at 181.61 101.6) (size 0.8) (drill 0.4) (layers F.Cu B.Cu) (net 4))
 (segment (start 181.61 102.885004) (end 154.955004 129.54) (width 0.25) (layer B.Cu) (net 4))
 (segment (start 181.61 101.6) (end 181.61 102.885004) (width 0.25) (layer B.Cu) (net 4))
 (segment (start 154.955004 129.54) (end 151.13 129.54) (width 0.25) (layer B.Cu) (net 4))
 (segment (start 151.13 129.54) (end 151.13 129.54) (width 0.25) (layer B.Cu) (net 4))
 (via (at 151.13 129.54) (size 0.8) (drill 0.4) (layers F.Cu B.Cu) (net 4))
 (segment (start 154.41 129.54) (end 155.68 128.27) (width 0.25) (layer F.Cu) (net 4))
 (segment (start 151.13 129.54) (end 154.41 129.54) (width 0.25) (layer F.Cu) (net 4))
 (segment (start 170.875001 123.19) (end 172.225001 123.19) (width 0.25) (layer F.Cu) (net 5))
 (segment (start 135.494998 123.19) (end 170.875001 123.19) (width 0.25) (layer F.Cu) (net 5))
 (segment (start 131.53499 127.150008) (end 135.494998 123.19) (width 0.25) (layer F.Cu) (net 5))
 (segment (start 131.53499 135.40818) (end 131.53499 127.150008) (width 0.25) (layer F.Cu) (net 5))
 (segment (start 133.55681 137.43) (end 131.53499 135.40818) (width 0.25) (layer F.Cu) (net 5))
 (segment (start 153.465 137.43) (end 133.55681 137.43) (width 0.25) (layer F.Cu) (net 5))
 (segment (start 122.93 139.7) (end 128.01 134.62) (width 0.25) (layer F.Cu) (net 6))
 (segment (start 116.84 139.7) (end 122.93 139.7) (width 0.25) (layer F.Cu) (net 6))
 (segment (start 131.32 137.93) (end 128.01 134.62) (width 0.25) (layer F.Cu) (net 6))
 (segment (start 153.465 137.93) (end 131.32 137.93) (width 0.25) (layer F.Cu) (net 6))
 (segment (start 153.465 137.93) (end 145.28 137.93) (width 0.25) (layer F.Cu) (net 6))
 (segment (start 145.28 137.93) (end 143.51 139.7) (width 0.25) (layer F.Cu) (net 6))
 (segment (start 143.51 139.7) (end 143.51 139.7) (width 0.25) (layer F.Cu) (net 6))
 (via (at 143.51 139.7) (size 0.8) (drill 0.4) (layers F.Cu B.Cu) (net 6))
 (segment (start 143.51 139.7) (end 148.59 134.62) (width 0.25) (layer B.Cu) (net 6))
 (segment (start 148.59 134.62) (end 154.94 134.62) (width 0.25) (layer B.Cu) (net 6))
 (segment (start 154.94 134.62) (end 154.94 134.62) (width 0.25) (layer B.Cu) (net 6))
 (via (at 154.94 134.62) (size 0.8) (drill 0.4) (layers F.Cu B.Cu) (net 6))
 (segment (start 156.415 136.095) (end 156.415 137.43) (width 0.25) (layer F.Cu) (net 6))
 (segment (start 154.94 134.62) (end 156.415 136.095) (width 0.25) (layer F.Cu) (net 6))
 (segment (start 175.73 87.47) (end 176.53 87.47) (width 0.25) (layer F.Cu) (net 7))
 (segment (start 148.59 138.43) (end 153.465 138.43) (width 0.25) (layer F.Cu) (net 8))
 (segment (start 146.05 140.97) (end 148.59 138.43) (width 0.25) (layer F.Cu) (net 8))
 (segment (start 190.5 99.06) (end 191.77 97.79) (width 0.25) (layer F.Cu) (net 9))
 (segment (start 190.5 113.67) (end 190.5 99.06) (width 0.25) (layer F.Cu) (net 9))
 (segment (start 156.415 138.93) (end 156.44999 138.89501) (width 0.25) (layer F.Cu) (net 10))
 (segment (start 156.415 138.93) (end 158.25 138.93) (width 0.25) (layer F.Cu) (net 10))
 (segment (start 158.25 138.93) (end 158.75 138.43) (width 0.25) (layer F.Cu) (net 10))
 (segment (start 158.75 138.43) (end 158.75 138.43) (width 0.25) (layer F.Cu) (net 10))
 (via (at 158.75 138.43) (size 0.8) (drill 0.4) (layers F.Cu B.Cu) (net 10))
 (segment (start 200.79863 99.06) (end 201.93 99.06) (width 0.25) (layer B.Cu) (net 10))
 (segment (start 191.966998 99.06) (end 200.79863 99.06) (width 0.25) (layer B.Cu) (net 10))
 (segment (start 158.024999 133.001999) (end 191.966998 99.06) (width 0.25) (layer B.Cu) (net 10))
 (segment (start 158.024999 137.704999) (end 158.024999 133.001999) (width 0.25) (layer B.Cu) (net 10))
 (segment (start 158.75 138.43) (end 158.024999 137.704999) (width 0.25) (layer B.Cu) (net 10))
 (segment (start 157.676998 133.35) (end 158.024999 133.001999) (width 0.25) (layer B.Cu) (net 10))
 (segment (start 148.59 133.35) (end 157.676998 133.35) (width 0.25) (layer B.Cu) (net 10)))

